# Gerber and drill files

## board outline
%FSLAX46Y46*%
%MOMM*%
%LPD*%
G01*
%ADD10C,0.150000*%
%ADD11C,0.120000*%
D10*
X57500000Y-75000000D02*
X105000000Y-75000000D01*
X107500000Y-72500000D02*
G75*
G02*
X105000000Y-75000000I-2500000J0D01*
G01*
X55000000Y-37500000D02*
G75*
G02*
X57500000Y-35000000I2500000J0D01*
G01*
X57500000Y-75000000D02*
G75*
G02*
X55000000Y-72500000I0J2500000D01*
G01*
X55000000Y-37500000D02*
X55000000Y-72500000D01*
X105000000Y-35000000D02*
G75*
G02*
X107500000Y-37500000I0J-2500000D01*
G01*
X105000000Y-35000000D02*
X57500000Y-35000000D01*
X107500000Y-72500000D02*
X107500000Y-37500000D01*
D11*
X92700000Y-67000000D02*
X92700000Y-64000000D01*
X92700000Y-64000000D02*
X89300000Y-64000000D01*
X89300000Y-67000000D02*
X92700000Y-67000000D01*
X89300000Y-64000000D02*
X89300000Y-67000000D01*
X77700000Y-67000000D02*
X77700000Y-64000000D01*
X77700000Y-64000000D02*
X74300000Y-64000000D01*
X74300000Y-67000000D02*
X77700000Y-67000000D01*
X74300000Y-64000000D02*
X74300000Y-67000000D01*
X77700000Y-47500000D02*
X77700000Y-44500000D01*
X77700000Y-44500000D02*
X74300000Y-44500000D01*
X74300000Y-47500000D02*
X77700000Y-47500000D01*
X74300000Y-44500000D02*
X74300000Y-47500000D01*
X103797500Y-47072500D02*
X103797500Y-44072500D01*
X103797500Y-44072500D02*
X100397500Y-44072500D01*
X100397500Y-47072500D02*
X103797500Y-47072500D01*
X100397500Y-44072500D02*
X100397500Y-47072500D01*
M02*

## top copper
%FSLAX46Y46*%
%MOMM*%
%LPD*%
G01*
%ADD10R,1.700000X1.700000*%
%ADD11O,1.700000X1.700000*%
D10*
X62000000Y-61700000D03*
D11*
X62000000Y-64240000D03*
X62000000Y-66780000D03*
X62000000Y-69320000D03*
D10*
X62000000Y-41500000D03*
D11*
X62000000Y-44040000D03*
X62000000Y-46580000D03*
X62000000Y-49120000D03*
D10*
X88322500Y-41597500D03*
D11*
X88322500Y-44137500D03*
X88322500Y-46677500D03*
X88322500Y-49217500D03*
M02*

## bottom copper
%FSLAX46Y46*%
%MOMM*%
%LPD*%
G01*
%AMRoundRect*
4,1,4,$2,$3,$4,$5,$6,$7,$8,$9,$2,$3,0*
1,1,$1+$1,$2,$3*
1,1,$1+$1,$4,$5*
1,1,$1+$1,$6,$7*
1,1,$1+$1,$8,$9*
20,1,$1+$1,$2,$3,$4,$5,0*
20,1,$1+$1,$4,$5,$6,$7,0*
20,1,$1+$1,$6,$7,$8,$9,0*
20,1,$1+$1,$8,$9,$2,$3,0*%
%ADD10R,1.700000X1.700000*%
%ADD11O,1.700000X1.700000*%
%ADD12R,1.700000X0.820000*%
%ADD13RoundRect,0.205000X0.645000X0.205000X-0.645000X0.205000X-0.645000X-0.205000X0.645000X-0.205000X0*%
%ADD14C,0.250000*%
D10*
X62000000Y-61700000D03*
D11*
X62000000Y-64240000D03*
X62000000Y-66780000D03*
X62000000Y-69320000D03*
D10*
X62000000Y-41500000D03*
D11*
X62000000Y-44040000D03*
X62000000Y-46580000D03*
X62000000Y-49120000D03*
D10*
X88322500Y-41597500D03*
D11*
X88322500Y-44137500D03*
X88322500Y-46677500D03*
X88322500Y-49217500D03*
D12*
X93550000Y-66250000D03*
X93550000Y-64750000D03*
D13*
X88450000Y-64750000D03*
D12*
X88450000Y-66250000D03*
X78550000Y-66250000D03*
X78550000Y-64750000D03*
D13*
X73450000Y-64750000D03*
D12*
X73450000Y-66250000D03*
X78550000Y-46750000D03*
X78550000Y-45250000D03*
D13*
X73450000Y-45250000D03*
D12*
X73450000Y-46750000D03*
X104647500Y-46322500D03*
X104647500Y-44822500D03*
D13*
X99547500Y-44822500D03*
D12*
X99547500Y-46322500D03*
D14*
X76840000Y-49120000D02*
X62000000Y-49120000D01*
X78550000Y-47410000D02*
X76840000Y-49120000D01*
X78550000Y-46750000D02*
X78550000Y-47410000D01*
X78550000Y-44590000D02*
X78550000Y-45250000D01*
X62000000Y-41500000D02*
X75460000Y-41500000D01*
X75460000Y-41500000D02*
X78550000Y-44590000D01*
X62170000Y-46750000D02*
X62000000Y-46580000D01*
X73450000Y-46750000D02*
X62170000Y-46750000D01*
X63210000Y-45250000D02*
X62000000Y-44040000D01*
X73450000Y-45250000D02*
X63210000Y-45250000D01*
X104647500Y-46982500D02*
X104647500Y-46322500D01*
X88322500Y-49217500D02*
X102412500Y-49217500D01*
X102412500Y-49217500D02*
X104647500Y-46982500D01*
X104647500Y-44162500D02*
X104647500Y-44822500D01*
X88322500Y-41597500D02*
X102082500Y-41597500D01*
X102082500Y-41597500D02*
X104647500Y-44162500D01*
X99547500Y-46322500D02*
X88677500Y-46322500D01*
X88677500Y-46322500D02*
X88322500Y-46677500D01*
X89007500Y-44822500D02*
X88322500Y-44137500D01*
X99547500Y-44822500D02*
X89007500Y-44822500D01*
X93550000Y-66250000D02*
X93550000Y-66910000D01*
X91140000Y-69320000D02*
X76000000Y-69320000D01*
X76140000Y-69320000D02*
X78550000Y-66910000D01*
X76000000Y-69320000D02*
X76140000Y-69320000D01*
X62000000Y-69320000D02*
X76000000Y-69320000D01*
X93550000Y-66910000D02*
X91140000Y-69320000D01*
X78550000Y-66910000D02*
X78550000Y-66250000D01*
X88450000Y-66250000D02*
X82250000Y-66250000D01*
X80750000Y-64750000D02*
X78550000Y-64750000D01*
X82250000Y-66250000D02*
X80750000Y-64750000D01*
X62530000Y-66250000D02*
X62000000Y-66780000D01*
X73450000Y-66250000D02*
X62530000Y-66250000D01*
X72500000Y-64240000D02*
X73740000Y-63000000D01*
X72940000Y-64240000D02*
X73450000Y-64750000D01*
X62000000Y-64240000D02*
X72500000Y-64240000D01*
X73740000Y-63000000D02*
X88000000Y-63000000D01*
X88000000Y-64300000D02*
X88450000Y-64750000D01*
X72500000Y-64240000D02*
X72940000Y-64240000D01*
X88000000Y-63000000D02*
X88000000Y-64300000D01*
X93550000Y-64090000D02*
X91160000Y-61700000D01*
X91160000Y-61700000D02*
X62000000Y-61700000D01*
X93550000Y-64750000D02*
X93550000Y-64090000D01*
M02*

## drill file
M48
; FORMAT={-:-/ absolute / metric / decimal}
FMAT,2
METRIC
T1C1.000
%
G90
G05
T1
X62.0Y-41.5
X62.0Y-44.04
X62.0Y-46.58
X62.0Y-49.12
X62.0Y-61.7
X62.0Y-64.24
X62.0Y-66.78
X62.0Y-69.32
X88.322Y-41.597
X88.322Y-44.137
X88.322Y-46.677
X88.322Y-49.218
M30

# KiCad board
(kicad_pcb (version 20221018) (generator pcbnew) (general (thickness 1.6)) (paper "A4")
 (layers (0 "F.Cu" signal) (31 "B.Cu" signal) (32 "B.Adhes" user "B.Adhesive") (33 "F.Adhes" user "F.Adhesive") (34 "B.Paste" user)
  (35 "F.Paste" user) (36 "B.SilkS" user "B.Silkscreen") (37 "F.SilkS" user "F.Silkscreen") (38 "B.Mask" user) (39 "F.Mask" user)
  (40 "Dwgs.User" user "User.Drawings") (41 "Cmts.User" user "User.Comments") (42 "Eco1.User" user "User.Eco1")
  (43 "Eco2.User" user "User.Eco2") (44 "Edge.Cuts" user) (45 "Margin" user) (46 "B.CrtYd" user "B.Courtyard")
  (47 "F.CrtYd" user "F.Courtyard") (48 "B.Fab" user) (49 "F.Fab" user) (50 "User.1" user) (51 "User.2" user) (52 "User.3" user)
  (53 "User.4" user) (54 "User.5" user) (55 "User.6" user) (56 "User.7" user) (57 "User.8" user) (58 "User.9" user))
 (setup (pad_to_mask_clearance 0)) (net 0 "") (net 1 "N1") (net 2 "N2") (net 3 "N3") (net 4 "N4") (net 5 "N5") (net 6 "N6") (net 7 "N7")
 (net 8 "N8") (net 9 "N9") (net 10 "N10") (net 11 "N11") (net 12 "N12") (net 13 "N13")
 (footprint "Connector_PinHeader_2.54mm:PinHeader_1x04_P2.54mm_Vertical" (layer "F.Cu") (at 62 61.7)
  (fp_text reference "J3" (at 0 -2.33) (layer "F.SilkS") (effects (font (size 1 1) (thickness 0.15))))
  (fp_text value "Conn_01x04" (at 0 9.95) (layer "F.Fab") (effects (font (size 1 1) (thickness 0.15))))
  (pad "1" thru_hole rect (at 0 0) (size 1.7 1.7) (drill 1) (layers "*.Cu" "*.Mask") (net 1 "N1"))
  (pad "2" thru_hole oval (at 0 2.54) (size 1.7 1.7) (drill 1) (layers "*.Cu" "*.Mask") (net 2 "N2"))
  (pad "3" thru_hole oval (at 0 5.08) (size 1.7 1.7) (drill 1) (layers "*.Cu" "*.Mask") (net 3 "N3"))
  (pad "4" thru_hole oval (at 0 7.62) (size 1.7 1.7) (drill 1) (layers "*.Cu" "*.Mask") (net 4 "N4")))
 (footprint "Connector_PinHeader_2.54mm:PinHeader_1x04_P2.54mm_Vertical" (layer "F.Cu") (at 62 41.5)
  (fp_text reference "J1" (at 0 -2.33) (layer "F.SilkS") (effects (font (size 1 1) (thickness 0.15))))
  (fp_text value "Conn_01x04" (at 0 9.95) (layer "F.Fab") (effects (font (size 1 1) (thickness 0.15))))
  (pad "1" thru_hole rect (at 0 0) (size 1.7 1.7) (drill 1) (layers "*.Cu" "*.Mask") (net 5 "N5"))
  (pad "2" thru_hole oval (at 0 2.54) (size 1.7 1.7) (drill 1) (layers "*.Cu" "*.Mask") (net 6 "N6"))
  (pad "3" thru_hole oval (at 0 5.08) (size 1.7 1.7) (drill 1) (layers "*.Cu" "*.Mask") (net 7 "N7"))
  (pad "4" thru_hole oval (at 0 7.62) (size 1.7 1.7) (drill 1) (layers "*.Cu" "*.Mask") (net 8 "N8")))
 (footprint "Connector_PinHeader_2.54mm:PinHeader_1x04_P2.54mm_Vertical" (layer "F.Cu") (at 88.3225 41.5975)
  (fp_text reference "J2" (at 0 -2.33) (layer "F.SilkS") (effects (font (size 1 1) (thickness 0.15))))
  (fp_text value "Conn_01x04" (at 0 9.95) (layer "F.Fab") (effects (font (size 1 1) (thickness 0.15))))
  (pad "1" thru_hole rect (at 0 0) (size 1.7 1.7) (drill 1) (layers "*.Cu" "*.Mask") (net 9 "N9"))
  (pad "2" thru_hole oval (at 0 2.54) (size 1.7 1.7) (drill 1) (layers "*.Cu" "*.Mask") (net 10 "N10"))
  (pad "3" thru_hole oval (at 0 5.08) (size 1.7 1.7) (drill 1) (layers "*.Cu" "*.Mask") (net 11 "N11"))
  (pad "4" thru_hole oval (at 0 7.62) (size 1.7 1.7) (drill 1) (layers "*.Cu" "*.Mask") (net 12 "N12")))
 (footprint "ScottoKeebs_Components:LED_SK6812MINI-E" (layer "B.Cu") (at 91 65.5 180)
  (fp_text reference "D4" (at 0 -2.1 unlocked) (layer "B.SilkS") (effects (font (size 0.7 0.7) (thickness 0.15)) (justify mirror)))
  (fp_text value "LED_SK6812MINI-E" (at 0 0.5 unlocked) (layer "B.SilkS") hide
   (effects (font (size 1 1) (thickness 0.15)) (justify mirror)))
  (fp_line (start -1.7 -1.5) (end -1.7 1.5) (stroke (width 0.12) (type solid)) (layer "Edge.Cuts"))
  (fp_line (start -1.7 1.5) (end 1.7 1.5) (stroke (width 0.12) (type solid)) (layer "Edge.Cuts"))
  (fp_line (start 1.7 -1.5) (end -1.7 -1.5) (stroke (width 0.12) (type solid)) (layer "Edge.Cuts"))
  (fp_line (start 1.7 1.5) (end 1.7 -1.5) (stroke (width 0.12) (type solid)) (layer "Edge.Cuts"))
  (pad "1" smd rect (at -2.55 -0.75 180) (size 1.7 0.82) (layers "B.Cu" "B.Paste" "B.Mask") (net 4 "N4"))
  (pad "2" smd rect (at -2.55 0.75 180) (size 1.7 0.82) (layers "B.Cu" "B.Paste" "B.Mask") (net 1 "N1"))
  (pad "3" smd roundrect (at 2.55 0.75 180) (size 1.7 0.82) (layers "B.Cu" "B.Paste" "B.Mask") (roundrect_rratio 0.25) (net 2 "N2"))
  (pad "4" smd rect (at 2.55 -0.75 180) (size 1.7 0.82) (layers "B.Cu" "B.Paste" "B.Mask") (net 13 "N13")))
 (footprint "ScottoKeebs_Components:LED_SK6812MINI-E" (layer "B.Cu") (at 76 65.5 180)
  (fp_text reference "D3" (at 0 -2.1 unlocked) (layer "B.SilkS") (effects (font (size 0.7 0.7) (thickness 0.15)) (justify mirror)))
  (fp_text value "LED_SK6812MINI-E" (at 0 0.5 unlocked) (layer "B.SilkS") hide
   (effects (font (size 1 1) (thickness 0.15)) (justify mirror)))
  (fp_line (start -1.7 -1.5) (end -1.7 1.5) (stroke (width 0.12) (type solid)) (layer "Edge.Cuts"))
  (fp_line (start -1.7 1.5) (end 1.7 1.5) (stroke (width 0.12) (type solid)) (layer "Edge.Cuts"))
  (fp_line (start 1.7 -1.5) (end -1.7 -1.5) (stroke (width 0.12) (type solid)) (layer "Edge.Cuts"))
  (fp_line (start 1.7 1.5) (end 1.7 -1.5) (stroke (width 0.12) (type solid)) (layer "Edge.Cuts"))
  (pad "1" smd rect (at -2.55 -0.75 180) (size 1.7 0.82) (layers "B.Cu" "B.Paste" "B.Mask") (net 4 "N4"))
  (pad "2" smd rect (at -2.55 0.75 180) (size 1.7 0.82) (layers "B.Cu" "B.Paste" "B.Mask") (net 13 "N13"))
  (pad "3" smd roundrect (at 2.55 0.75 180) (size 1.7 0.82) (layers "B.Cu" "B.Paste" "B.Mask") (roundrect_rratio 0.25) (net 2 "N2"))
  (pad "4" smd rect (at 2.55 -0.75 180) (size 1.7 0.82) (layers "B.Cu" "B.Paste" "B.Mask") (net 3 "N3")))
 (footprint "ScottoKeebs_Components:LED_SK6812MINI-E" (layer "B.Cu") (at 76 46 180)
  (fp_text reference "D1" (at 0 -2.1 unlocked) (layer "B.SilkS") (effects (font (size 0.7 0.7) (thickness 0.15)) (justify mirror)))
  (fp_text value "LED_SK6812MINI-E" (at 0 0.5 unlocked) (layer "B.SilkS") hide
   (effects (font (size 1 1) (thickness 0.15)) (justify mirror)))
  (fp_line (start -1.7 -1.5) (end -1.7 1.5) (stroke (width 0.12) (type solid)) (layer "Edge.Cuts"))
  (fp_line (start -1.7 1.5) (end 1.7 1.5) (stroke (width 0.12) (type solid)) (layer "Edge.Cuts"))
  (fp_line (start 1.7 -1.5) (end -1.7 -1.5) (stroke (width 0.12) (type solid)) (layer "Edge.Cuts"))
  (fp_line (start 1.7 1.5) (end 1.7 -1.5) (stroke (width 0.12) (type solid)) (layer "Edge.Cuts"))
  (pad "1" smd rect (at -2.55 -0.75 180) (size 1.7 0.82) (layers "B.Cu" "B.Paste" "B.Mask") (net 8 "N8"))
  (pad "2" smd rect (at -2.55 0.75 180) (size 1.7 0.82) (layers "B.Cu" "B.Paste" "B.Mask") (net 5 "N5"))
  (pad "3" smd roundrect (at 2.55 0.75 180) (size 1.7 0.82) (layers "B.Cu" "B.Paste" "B.Mask") (roundrect_rratio 0.25) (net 6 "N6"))
  (pad "4" smd rect (at 2.55 -0.75 180) (size 1.7 0.82) (layers "B.Cu" "B.Paste" "B.Mask") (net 7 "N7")))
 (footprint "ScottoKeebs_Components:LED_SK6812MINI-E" (layer "B.Cu") (at 102.0975 45.5725 180)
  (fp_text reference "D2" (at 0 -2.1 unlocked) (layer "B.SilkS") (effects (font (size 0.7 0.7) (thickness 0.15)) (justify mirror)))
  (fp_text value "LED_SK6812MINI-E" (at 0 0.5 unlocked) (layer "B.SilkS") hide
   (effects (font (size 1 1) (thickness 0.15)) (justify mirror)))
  (fp_line (start -1.7 -1.5) (end -1.7 1.5) (stroke (width 0.12) (type solid)) (layer "Edge.Cuts"))
  (fp_line (start -1.7 1.5) (end 1.7 1.5) (stroke (width 0.12) (type solid)) (layer "Edge.Cuts"))
  (fp_line (start 1.7 -1.5) (end -1.7 -1.5) (stroke (width 0.12) (type solid)) (layer "Edge.Cuts"))
  (fp_line (start 1.7 1.5) (end 1.7 -1.5) (stroke (width 0.12) (type solid)) (layer "Edge.Cuts"))
  (pad "1" smd rect (at -2.55 -0.75 180) (size 1.7 0.82) (layers "B.Cu" "B.Paste" "B.Mask") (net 12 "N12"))
  (pad "2" smd rect (at -2.55 0.75 180) (size 1.7 0.82) (layers "B.Cu" "B.Paste" "B.Mask") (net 9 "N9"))
  (pad "3" smd roundrect (at 2.55 0.75 180) (size 1.7 0.82) (layers "B.Cu" "B.Paste" "B.Mask") (roundrect_rratio 0.25) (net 10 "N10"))
  (pad "4" smd rect (at 2.55 -0.75 180) (size 1.7 0.82) (layers "B.Cu" "B.Paste" "B.Mask") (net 11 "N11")))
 (gr_line (start 57.5 75) (end 105 75) (stroke (width 0.15) (type default)) (layer "Edge.Cuts"))
 (gr_arc (start 107.5 72.5) (mid 106.767767 74.267766) (end 105 75) (stroke (width 0.15) (type default)) (layer "Edge.Cuts"))
 (gr_arc (start 55 37.5) (mid 55.732233 35.732234) (end 57.5 35) (stroke (width 0.15) (type default)) (layer "Edge.Cuts"))
 (gr_arc (start 57.5 75) (mid 55.732234 74.267767) (end 55 72.5) (stroke (width 0.15) (type default)) (layer "Edge.Cuts"))
 (gr_line (start 55 37.5) (end 55 72.5) (stroke (width 0.15) (type default)) (layer "Edge.Cuts"))
 (gr_arc (start 105 35) (mid 106.767766 35.732233) (end 107.5 37.5) (stroke (width 0.15) (type default)) (layer "Edge.Cuts"))
 (gr_line (start 105 35) (end 57.5 35) (stroke (width 0.15) (type default)) (layer "Edge.Cuts"))
 (gr_line (start 107.5 72.5) (end 107.5 37.5) (stroke (width 0.15) (type default)) (layer "Edge.Cuts"))
 (segment (start 76.84 49.12) (end 62 49.12) (width 0.25) (layer "B.Cu") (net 8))
 (segment (start 78.55 47.41) (end 76.84 49.12) (width 0.25) (layer "B.Cu") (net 8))
 (segment (start 78.55 46.75) (end 78.55 47.41) (width 0.25) (layer "B.Cu") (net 8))
 (segment (start 78.55 44.59) (end 78.55 45.25) (width 0.25) (layer "B.Cu") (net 5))
 (segment (start 62 41.5) (end 75.46 41.5) (width 0.25) (layer "B.Cu") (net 5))
 (segment (start 75.46 41.5) (end 78.55 44.59) (width 0.25) (layer "B.Cu") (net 5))
 (segment (start 62.17 46.75) (end 62 46.58) (width 0.25) (layer "B.Cu") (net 7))
 (segment (start 73.45 46.75) (end 62.17 46.75) (width 0.25) (layer "B.Cu") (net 7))
 (segment (start 63.21 45.25) (end 62 44.04) (width 0.25) (layer "B.Cu") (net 6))
 (segment (start 73.45 45.25) (end 63.21 45.25) (width 0.25) (layer "B.Cu") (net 6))
 (segment (start 104.6475 46.9825) (end 104.6475 46.3225) (width 0.25) (layer "B.Cu") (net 12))
 (segment (start 88.3225 49.2175) (end 102.4125 49.2175) (width 0.25) (layer "B.Cu") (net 12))
 (segment (start 102.4125 49.2175) (end 104.6475 46.9825) (width 0.25) (layer "B.Cu") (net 12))
 (segment (start 104.6475 44.1625) (end 104.6475 44.8225) (width 0.25) (layer "B.Cu") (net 9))
 (segment (start 88.3225 41.5975) (end 102.0825 41.5975) (width 0.25) (layer "B.Cu") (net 9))
 (segment (start 102.0825 41.5975) (end 104.6475 44.1625) (width 0.25) (layer "B.Cu") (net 9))
 (segment (start 99.5475 46.3225) (end 88.6775 46.3225) (width 0.25) (layer "B.Cu") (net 11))
 (segment (start 88.6775 46.3225) (end 88.3225 46.6775) (width 0.25) (layer "B.Cu") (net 11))
 (segment (start 89.0075 44.8225) (end 88.3225 44.1375) (width 0.25) (layer "B.Cu") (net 10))
 (segment (start 99.5475 44.8225) (end 89.0075 44.8225) (width 0.25) (layer "B.Cu") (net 10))
 (segment (start 93.55 66.25) (end 93.55 66.91) (width 0.25) (layer "B.Cu") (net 4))
 (segment (start 91.14 69.32) (end 76 69.32) (width 0.25) (layer "B.Cu") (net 4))
 (segment (start 76.14 69.32) (end 78.55 66.91) (width 0.25) (layer "B.Cu") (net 4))
 (segment (start 76 69.32) (end 76.14 69.32) (width 0.25) (layer "B.Cu") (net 4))
 (segment (start 62 69.32) (end 76 69.32) (width 0.25) (layer "B.Cu") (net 4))
 (segment (start 93.55 66.91) (end 91.14 69.32) (width 0.25) (layer "B.Cu") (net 4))
 (segment (start 78.55 66.91) (end 78.55 66.25) (width 0.25) (layer "B.Cu") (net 4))
 (segment (start 88.45 66.25) (end 82.25 66.25) (width 0.25) (layer "B.Cu") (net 13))
 (segment (start 80.75 64.75) (end 78.55 64.75) (width 0.25) (layer "B.Cu") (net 13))
 (segment (start 82.25 66.25) (end 80.75 64.75) (width 0.25) (layer "B.Cu") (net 13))
 (segment (start 62.53 66.25) (end 62 66.78) (width 0.25) (layer "B.Cu") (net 3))
 (segment (start 73.45 66.25) (end 62.53 66.25) (width 0.25) (layer "B.Cu") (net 3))
 (segment (start 72.5 64.24) (end 73.74 63) (width 0.25) (layer "B.Cu") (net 2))
 (segment (start 72.94 64.24) (end 73.45 64.75) (width 0.25) (layer "B.Cu") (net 2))
 (segment (start 62 64.24) (end 72.5 64.24) (width 0.25) (layer "B.Cu") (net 2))
 (segment (start 73.74 63) (end 88 63) (width 0.25) (layer "B.Cu") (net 2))
 (segment (start 88 64.3) (end 88.45 64.75) (width 0.25) (layer "B.Cu") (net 2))
 (segment (start 72.5 64.24) (end 72.94 64.24) (width 0.25) (layer "B.Cu") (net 2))
 (segment (start 88 63) (end 88 64.3) (width 0.25) (layer "B.Cu") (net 2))
 (segment (start 93.55 64.09) (end 91.16 61.7) (width 0.25) (layer "B.Cu") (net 1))
 (segment (start 91.16 61.7) (end 62 61.7) (width 0.25) (layer "B.Cu") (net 1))
 (segment (start 93.55 64.75) (end 93.55 64.09) (width 0.25) (layer "B.Cu") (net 1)))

